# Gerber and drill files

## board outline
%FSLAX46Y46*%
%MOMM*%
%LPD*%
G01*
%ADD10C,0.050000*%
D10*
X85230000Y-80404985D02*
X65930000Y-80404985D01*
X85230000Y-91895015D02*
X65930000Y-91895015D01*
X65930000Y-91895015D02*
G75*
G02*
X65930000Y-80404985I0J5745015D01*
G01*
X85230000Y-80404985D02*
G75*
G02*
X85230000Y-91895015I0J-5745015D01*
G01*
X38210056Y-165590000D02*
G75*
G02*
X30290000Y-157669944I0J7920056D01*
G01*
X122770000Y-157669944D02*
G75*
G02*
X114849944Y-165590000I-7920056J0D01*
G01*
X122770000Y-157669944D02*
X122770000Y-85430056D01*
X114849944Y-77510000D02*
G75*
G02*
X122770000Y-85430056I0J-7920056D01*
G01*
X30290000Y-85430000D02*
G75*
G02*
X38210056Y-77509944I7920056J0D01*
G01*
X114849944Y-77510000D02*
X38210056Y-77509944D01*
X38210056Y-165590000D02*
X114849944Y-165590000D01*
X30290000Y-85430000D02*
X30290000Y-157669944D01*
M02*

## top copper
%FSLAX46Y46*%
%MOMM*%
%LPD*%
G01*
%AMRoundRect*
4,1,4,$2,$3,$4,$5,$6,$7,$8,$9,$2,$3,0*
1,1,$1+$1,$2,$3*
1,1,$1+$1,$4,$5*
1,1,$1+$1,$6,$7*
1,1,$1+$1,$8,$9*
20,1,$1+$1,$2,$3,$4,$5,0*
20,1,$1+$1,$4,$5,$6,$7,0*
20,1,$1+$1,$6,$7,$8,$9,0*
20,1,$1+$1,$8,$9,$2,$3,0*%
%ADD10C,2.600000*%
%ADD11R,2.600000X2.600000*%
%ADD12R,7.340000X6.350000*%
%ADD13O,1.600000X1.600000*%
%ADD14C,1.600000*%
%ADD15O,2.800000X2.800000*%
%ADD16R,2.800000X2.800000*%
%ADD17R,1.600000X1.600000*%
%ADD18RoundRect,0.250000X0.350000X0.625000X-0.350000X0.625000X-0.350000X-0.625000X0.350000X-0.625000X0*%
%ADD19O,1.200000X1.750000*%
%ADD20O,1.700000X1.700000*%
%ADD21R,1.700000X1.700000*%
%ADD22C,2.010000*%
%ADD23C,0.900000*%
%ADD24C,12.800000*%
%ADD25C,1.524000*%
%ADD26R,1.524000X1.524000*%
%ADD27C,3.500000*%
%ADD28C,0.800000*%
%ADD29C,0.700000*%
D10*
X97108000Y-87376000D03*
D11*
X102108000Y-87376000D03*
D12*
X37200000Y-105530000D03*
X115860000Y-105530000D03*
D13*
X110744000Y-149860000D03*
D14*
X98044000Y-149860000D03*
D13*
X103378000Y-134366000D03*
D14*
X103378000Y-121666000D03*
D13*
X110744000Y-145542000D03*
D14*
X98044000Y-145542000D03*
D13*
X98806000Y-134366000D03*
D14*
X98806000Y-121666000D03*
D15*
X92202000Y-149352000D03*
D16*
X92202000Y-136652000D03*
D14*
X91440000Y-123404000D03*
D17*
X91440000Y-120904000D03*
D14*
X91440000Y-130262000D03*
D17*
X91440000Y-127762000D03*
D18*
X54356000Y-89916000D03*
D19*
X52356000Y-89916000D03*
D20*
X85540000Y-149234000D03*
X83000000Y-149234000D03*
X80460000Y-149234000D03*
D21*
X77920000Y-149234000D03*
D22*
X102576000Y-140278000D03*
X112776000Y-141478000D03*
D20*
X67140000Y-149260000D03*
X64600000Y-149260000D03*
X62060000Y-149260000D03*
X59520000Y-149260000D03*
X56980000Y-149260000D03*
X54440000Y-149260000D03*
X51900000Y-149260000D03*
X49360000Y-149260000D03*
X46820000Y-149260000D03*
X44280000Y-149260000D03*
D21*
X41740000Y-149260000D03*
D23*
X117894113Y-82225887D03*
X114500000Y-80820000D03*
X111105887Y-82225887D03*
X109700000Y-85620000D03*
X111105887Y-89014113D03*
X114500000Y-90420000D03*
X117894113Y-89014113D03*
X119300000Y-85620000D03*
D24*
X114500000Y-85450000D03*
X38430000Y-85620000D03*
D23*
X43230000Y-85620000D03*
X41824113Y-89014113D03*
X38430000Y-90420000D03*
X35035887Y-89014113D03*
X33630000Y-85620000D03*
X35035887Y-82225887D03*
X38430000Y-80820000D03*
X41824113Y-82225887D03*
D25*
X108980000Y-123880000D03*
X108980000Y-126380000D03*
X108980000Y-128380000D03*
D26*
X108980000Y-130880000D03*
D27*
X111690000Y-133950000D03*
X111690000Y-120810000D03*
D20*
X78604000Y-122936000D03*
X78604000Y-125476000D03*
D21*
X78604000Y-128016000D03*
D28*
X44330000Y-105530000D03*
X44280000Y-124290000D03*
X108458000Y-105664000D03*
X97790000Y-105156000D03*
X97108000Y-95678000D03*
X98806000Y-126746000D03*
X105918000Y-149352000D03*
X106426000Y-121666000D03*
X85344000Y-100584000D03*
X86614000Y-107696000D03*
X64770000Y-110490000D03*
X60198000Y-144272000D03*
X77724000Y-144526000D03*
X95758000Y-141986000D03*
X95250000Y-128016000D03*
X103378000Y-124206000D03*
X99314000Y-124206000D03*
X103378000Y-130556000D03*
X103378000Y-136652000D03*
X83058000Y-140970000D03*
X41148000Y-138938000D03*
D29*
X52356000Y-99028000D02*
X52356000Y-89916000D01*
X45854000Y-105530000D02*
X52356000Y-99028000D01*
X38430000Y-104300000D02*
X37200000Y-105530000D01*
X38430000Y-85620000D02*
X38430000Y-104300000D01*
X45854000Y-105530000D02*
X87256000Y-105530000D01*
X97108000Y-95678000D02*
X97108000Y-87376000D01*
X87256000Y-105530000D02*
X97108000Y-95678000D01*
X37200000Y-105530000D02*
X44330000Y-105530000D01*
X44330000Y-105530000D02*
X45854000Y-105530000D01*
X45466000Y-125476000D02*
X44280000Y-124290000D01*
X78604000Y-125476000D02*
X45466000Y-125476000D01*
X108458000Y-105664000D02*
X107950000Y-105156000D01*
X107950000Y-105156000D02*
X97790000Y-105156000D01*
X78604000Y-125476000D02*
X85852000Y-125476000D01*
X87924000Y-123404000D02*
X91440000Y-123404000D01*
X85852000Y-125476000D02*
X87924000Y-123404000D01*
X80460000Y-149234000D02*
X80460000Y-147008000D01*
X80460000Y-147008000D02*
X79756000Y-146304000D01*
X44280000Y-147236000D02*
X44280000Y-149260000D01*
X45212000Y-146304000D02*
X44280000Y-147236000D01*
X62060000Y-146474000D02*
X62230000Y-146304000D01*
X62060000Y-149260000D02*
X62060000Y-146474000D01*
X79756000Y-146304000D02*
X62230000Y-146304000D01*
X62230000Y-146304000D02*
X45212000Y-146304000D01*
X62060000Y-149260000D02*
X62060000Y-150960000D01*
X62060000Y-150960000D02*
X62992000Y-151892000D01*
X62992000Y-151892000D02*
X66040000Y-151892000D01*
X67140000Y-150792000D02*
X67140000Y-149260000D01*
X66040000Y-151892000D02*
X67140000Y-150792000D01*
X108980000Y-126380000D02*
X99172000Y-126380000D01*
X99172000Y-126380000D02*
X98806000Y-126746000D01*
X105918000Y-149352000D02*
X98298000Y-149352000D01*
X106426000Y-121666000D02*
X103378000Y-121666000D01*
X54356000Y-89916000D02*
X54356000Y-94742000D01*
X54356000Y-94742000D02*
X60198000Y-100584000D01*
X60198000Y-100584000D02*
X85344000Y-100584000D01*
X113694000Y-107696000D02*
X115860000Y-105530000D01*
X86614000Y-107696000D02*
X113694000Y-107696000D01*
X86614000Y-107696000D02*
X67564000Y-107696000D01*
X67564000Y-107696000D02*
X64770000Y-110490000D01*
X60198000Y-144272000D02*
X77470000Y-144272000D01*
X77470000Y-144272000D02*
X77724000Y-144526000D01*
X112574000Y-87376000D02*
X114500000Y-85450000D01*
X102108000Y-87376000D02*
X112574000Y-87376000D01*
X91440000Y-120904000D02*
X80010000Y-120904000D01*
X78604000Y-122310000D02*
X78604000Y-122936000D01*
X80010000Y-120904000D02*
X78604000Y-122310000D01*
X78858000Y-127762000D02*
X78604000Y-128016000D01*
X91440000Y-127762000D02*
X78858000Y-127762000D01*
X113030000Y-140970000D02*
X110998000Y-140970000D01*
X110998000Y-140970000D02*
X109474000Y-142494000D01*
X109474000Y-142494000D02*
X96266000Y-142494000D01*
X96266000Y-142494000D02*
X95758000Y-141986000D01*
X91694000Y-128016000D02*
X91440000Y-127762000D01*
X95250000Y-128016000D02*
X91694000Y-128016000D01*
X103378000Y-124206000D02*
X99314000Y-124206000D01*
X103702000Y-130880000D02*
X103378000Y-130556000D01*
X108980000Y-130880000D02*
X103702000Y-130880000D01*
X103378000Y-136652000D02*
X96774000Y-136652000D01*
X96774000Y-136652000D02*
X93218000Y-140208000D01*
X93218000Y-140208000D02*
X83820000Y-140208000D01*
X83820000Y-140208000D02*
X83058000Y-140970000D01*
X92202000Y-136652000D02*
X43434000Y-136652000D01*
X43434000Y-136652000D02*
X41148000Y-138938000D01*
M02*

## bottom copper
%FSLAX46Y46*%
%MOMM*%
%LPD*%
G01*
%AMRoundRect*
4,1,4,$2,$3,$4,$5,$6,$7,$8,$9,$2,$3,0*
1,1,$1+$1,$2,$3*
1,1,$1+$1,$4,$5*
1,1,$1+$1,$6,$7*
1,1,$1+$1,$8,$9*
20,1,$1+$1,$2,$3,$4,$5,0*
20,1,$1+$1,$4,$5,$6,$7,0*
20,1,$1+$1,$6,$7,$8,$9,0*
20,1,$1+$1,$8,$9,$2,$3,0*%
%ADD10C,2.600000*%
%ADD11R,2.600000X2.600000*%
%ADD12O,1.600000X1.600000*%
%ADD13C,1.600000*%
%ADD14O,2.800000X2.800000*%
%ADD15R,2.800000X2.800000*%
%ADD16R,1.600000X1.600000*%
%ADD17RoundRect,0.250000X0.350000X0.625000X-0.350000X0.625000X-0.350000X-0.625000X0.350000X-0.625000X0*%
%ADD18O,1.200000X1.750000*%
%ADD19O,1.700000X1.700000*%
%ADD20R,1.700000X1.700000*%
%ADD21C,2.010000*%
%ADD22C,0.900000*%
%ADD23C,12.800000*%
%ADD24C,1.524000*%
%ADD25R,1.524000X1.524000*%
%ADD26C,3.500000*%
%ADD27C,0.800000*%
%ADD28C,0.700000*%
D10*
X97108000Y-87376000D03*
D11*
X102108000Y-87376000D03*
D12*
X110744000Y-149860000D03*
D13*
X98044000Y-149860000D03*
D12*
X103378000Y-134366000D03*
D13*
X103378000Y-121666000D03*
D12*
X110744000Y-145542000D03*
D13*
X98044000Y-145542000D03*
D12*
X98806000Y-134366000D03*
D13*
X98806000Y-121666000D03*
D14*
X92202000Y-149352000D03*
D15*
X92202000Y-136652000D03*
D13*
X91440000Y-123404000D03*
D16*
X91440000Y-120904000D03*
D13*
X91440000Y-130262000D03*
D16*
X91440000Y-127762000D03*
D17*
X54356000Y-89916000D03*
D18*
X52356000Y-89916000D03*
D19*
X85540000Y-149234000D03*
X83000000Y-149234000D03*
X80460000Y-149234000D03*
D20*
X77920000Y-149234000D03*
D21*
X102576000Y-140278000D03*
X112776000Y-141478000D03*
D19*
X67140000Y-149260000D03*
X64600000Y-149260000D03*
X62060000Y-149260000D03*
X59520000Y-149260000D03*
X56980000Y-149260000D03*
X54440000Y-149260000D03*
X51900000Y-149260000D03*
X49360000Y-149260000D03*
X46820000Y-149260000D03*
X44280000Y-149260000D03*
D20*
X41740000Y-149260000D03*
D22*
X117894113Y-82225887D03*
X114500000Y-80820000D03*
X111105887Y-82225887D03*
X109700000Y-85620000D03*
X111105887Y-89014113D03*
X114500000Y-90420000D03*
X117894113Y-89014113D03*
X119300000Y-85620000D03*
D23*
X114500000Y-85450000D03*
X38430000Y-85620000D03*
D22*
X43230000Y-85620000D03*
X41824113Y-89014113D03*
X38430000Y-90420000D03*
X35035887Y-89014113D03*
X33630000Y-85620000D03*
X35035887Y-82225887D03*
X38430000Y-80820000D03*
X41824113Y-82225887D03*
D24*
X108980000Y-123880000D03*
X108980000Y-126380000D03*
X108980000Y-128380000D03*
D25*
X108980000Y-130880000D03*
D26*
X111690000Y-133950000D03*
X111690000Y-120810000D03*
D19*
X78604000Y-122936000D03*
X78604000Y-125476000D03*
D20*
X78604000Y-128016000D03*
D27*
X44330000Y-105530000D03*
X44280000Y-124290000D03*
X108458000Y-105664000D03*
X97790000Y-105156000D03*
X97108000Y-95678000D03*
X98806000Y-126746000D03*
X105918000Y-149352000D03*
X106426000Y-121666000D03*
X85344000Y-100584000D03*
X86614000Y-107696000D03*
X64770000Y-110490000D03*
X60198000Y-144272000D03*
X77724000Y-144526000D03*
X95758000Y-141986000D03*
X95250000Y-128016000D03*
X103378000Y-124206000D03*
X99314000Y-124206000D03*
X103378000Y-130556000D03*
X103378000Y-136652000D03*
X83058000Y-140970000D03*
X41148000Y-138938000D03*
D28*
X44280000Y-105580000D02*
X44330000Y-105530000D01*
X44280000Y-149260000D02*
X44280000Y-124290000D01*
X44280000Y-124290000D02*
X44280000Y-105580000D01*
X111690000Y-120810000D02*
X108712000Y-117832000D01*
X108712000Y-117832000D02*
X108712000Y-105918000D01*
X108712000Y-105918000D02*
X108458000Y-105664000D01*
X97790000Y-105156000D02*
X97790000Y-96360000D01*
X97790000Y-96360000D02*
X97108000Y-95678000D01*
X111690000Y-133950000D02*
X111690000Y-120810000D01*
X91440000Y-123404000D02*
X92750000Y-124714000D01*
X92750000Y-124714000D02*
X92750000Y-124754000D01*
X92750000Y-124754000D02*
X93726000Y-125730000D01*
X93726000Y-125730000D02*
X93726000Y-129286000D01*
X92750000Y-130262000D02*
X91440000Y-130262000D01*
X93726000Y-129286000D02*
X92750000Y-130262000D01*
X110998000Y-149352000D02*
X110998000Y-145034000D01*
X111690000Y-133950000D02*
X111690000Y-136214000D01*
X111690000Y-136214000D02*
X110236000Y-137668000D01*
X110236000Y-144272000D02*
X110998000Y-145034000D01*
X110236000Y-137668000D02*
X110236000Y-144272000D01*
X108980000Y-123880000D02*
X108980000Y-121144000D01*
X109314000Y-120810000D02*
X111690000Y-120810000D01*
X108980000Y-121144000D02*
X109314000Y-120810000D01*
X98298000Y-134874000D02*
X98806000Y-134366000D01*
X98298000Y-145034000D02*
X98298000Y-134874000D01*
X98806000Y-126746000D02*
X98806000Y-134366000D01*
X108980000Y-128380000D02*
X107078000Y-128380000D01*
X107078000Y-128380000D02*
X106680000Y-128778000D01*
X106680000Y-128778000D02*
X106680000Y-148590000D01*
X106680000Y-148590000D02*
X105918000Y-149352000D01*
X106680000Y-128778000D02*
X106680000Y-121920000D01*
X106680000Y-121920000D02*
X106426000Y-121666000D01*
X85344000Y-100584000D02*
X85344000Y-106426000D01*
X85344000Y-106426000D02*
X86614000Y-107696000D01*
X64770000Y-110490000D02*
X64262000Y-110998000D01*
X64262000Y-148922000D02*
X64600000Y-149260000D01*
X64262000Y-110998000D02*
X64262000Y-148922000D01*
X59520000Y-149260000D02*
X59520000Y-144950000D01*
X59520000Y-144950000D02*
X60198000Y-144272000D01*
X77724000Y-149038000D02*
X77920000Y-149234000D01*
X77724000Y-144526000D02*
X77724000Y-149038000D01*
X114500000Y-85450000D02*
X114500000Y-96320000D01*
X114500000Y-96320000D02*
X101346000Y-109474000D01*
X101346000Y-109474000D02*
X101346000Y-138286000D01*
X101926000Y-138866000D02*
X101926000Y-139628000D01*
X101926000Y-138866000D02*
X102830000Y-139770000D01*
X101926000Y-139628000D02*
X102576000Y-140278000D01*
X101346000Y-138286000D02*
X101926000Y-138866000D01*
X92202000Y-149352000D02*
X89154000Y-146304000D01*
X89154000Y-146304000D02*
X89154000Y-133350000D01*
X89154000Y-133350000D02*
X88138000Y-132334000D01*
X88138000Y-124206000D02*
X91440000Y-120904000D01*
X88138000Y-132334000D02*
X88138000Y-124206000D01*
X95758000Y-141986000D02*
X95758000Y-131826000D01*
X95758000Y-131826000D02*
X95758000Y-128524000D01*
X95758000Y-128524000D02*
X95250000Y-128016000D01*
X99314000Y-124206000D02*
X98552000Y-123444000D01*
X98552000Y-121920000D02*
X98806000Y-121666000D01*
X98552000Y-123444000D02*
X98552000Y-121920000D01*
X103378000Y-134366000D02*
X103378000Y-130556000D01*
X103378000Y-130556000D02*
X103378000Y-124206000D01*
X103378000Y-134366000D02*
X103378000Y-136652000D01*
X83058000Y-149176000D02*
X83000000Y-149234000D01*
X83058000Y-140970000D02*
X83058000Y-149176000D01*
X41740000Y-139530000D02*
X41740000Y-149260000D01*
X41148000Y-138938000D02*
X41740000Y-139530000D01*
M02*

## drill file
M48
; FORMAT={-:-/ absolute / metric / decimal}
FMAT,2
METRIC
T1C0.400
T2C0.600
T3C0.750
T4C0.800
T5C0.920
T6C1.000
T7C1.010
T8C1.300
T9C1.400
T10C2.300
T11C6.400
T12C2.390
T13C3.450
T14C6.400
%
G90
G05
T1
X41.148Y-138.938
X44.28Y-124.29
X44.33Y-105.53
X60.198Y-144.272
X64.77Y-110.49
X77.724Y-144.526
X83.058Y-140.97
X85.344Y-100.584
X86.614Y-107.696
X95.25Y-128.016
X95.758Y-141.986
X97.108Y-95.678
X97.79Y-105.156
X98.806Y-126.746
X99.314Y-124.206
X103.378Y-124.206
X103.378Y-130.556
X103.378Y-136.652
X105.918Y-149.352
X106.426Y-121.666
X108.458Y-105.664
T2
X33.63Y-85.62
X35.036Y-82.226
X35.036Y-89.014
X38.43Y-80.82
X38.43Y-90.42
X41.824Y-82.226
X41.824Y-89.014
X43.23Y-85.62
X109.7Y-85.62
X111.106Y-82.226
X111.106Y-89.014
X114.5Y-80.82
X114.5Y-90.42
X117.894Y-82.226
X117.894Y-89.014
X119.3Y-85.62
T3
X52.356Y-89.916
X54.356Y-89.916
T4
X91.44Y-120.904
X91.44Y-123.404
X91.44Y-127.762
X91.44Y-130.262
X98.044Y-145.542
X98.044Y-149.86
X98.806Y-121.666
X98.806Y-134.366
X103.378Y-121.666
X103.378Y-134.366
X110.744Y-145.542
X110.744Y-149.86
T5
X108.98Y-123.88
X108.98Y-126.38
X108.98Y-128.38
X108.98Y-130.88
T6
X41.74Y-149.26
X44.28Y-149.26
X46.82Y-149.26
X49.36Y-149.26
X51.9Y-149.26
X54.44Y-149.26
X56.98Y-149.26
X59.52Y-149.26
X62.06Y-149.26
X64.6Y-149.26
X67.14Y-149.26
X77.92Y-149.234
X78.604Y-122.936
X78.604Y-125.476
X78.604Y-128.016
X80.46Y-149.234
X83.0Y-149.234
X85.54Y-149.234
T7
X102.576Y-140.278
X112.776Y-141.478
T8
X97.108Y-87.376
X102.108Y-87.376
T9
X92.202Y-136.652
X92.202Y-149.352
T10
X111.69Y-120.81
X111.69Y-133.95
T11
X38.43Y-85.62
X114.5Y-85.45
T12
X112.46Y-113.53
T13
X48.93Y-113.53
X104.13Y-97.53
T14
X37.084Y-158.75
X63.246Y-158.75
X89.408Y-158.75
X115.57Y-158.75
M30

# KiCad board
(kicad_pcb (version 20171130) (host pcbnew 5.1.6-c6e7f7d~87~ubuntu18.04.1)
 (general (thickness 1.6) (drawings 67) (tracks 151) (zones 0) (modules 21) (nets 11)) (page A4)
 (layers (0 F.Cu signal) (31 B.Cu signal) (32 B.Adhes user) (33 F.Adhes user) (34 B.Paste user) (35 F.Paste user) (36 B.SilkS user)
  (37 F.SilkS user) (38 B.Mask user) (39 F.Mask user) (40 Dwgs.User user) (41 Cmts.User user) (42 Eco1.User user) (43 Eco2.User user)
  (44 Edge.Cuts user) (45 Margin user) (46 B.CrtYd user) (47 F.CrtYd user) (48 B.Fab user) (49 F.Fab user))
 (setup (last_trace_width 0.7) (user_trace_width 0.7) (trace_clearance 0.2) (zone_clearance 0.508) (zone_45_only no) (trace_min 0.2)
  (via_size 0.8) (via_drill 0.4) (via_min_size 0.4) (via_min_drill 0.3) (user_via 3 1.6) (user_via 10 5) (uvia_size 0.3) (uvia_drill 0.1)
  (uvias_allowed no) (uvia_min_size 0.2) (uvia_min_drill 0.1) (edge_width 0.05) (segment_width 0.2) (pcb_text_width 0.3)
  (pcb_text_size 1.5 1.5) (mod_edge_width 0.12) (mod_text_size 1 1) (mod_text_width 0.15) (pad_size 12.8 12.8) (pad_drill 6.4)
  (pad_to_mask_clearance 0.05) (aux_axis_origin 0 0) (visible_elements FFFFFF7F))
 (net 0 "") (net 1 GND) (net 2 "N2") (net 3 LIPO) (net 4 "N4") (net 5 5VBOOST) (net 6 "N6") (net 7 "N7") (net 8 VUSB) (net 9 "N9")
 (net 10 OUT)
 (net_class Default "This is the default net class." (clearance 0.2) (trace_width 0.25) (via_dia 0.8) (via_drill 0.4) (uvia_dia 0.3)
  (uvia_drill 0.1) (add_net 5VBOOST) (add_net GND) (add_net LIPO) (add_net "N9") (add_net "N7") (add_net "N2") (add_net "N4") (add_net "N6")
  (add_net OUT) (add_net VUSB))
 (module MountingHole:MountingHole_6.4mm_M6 (layer F.Cu) (at 89.408 158.75)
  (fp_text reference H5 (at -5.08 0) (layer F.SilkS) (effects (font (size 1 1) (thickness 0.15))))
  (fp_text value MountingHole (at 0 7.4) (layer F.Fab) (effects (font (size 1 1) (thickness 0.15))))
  (pad 1 np_thru_hole circle (at 0 0) (size 6.4 6.4) (drill 6.4) (layers *.Cu *.Mask)))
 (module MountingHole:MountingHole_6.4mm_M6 (layer F.Cu) (at 63.246 158.75)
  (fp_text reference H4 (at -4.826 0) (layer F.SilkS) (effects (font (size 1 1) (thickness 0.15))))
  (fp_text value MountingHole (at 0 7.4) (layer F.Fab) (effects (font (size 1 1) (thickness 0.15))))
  (pad 1 np_thru_hole circle (at 0 0) (size 6.4 6.4) (drill 6.4) (layers *.Cu *.Mask)))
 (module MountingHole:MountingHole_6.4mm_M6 (layer F.Cu) (at 115.57 158.75)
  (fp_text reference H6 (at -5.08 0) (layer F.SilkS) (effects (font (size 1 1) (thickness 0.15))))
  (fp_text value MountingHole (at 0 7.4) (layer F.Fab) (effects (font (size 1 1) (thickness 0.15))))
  (pad 1 np_thru_hole circle (at 0 0) (size 6.4 6.4) (drill 6.4) (layers *.Cu *.Mask)))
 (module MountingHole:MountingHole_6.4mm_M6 (layer F.Cu) (at 37.084 158.75)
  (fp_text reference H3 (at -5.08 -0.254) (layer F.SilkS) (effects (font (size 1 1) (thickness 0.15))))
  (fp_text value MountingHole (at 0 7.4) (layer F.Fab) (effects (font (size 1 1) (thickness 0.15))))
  (pad 1 np_thru_hole circle (at 0 0) (size 6.4 6.4) (drill 6.4) (layers *.Cu *.Mask)))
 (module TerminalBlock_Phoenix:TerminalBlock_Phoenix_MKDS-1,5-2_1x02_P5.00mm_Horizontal (layer F.Cu) (at 102.108 87.376 180)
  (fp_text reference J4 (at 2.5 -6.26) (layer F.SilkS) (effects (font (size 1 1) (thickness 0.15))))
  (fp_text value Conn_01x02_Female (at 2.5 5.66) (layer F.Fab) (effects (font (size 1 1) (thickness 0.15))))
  (pad 2 thru_hole circle (at 5 0 180) (size 2.6 2.6) (drill 1.3) (layers *.Cu *.Mask) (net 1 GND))
  (pad 1 thru_hole rect (at 0 0 180) (size 2.6 2.6) (drill 1.3) (layers *.Cu *.Mask) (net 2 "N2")))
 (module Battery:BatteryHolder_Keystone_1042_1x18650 (layer F.Cu) (at 76.53 105.53 180)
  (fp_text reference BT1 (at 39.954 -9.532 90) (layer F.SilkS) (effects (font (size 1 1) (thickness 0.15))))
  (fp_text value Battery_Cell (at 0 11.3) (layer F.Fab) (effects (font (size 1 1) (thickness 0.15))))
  (pad "" np_thru_hole circle (at -35.93 -8 180) (size 2.39 2.39) (drill 2.39) (layers *.Cu *.Mask))
  (pad "" np_thru_hole circle (at -27.6 8 180) (size 3.45 3.45) (drill 3.45) (layers *.Cu *.Mask))
  (pad "" np_thru_hole circle (at 27.6 -8 180) (size 3.45 3.45) (drill 3.45) (layers *.Cu *.Mask))
  (pad 2 smd rect (at 39.33 0 180) (size 7.34 6.35) (layers F.Cu F.Paste F.Mask) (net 1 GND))
  (pad 1 smd rect (at -39.33 0 180) (size 7.34 6.35) (layers F.Cu F.Paste F.Mask) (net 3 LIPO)))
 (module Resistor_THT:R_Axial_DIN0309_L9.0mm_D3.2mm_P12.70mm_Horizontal (layer F.Cu) (at 98.044 149.86)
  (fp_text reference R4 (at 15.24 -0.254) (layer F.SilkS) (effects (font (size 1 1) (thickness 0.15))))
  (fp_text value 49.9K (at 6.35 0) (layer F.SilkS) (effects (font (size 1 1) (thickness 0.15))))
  (pad 2 thru_hole oval (at 12.7 0) (size 1.6 1.6) (drill 0.8) (layers *.Cu *.Mask) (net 1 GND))
  (pad 1 thru_hole circle (at 0 0) (size 1.6 1.6) (drill 0.8) (layers *.Cu *.Mask) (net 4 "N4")))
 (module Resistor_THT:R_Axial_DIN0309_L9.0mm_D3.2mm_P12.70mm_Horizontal (layer F.Cu) (at 103.378 121.666 270)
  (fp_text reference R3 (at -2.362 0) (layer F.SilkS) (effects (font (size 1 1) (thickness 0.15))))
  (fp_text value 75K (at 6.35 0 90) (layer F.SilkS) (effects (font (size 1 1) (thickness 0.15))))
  (pad 2 thru_hole oval (at 12.7 0 270) (size 1.6 1.6) (drill 0.8) (layers *.Cu *.Mask) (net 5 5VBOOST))
  (pad 1 thru_hole circle (at 0 0 270) (size 1.6 1.6) (drill 0.8) (layers *.Cu *.Mask) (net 4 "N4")))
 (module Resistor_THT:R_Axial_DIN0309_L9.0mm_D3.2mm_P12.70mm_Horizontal (layer F.Cu) (at 98.044 145.542)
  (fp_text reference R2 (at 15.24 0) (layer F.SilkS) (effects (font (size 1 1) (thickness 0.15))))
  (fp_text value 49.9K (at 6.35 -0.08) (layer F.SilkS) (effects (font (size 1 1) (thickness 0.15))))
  (pad 2 thru_hole oval (at 12.7 0) (size 1.6 1.6) (drill 0.8) (layers *.Cu *.Mask) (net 1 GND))
  (pad 1 thru_hole circle (at 0 0) (size 1.6 1.6) (drill 0.8) (layers *.Cu *.Mask) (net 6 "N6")))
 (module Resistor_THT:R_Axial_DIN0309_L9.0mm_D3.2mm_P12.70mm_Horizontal (layer F.Cu) (at 98.806 121.666 270)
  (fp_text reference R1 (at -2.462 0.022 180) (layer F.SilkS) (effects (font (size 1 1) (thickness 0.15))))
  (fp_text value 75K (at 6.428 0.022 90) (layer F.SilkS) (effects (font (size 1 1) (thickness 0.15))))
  (pad 2 thru_hole oval (at 12.7 0 270) (size 1.6 1.6) (drill 0.8) (layers *.Cu *.Mask) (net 6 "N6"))
  (pad 1 thru_hole circle (at 0 0 270) (size 1.6 1.6) (drill 0.8) (layers *.Cu *.Mask) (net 5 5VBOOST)))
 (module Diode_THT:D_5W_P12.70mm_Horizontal (layer F.Cu) (at 92.202 136.652 270)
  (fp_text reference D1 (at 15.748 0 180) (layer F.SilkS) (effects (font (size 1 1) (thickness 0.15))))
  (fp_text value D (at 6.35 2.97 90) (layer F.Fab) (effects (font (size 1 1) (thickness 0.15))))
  (pad 2 thru_hole oval (at 12.7 0 270) (size 2.8 2.8) (drill 1.4) (layers *.Cu *.Mask) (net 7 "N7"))
  (pad 1 thru_hole rect (at 0 0 270) (size 2.8 2.8) (drill 1.4) (layers *.Cu *.Mask) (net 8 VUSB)))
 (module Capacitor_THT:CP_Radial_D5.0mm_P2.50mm (layer F.Cu) (at 91.44 120.904 270)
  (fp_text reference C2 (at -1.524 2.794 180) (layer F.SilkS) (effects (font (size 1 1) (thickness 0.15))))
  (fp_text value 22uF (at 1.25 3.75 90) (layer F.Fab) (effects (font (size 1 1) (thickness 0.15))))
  (pad 2 thru_hole circle (at 2.5 0 270) (size 1.6 1.6) (drill 0.8) (layers *.Cu *.Mask) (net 1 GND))
  (pad 1 thru_hole rect (at 0 0 270) (size 1.6 1.6) (drill 0.8) (layers *.Cu *.Mask) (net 7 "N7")))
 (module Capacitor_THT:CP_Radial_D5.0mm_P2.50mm (layer F.Cu) (at 91.44 127.762 270)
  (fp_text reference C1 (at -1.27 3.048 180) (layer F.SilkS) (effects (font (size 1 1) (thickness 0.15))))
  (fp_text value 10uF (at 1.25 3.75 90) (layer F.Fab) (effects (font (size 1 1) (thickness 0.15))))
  (pad 2 thru_hole circle (at 2.5 0 270) (size 1.6 1.6) (drill 0.8) (layers *.Cu *.Mask) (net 1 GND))
  (pad 1 thru_hole rect (at 0 0 270) (size 1.6 1.6) (drill 0.8) (layers *.Cu *.Mask) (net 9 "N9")))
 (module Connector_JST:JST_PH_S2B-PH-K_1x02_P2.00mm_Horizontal (layer F.Cu) (at 54.356 89.916 180)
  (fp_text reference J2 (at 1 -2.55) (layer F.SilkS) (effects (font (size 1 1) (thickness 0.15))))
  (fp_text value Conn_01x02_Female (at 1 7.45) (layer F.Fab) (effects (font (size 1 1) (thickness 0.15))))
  (pad 1 thru_hole roundrect (at 0 0 180) (size 1.2 1.75) (drill 0.75) (layers *.Cu *.Mask) (roundrect_rratio 0.208333) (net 3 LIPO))
  (pad 2 thru_hole oval (at 2 0 180) (size 1.2 1.75) (drill 0.75) (layers *.Cu *.Mask) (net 1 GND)))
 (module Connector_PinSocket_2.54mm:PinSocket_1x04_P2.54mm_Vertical (layer F.Cu) (at 77.92 149.234 90)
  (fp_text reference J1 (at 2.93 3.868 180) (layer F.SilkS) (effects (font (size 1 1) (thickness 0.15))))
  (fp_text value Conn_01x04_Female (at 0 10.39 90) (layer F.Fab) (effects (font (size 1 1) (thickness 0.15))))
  (pad 4 thru_hole oval (at 0 7.62 90) (size 1.7 1.7) (drill 1) (layers *.Cu *.Mask))
  (pad 3 thru_hole oval (at 0 5.08 90) (size 1.7 1.7) (drill 1) (layers *.Cu *.Mask) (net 5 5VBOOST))
  (pad 2 thru_hole oval (at 0 2.54 90) (size 1.7 1.7) (drill 1) (layers *.Cu *.Mask) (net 1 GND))
  (pad 1 thru_hole rect (at 0 0 90) (size 1.7 1.7) (drill 1) (layers *.Cu *.Mask) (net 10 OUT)))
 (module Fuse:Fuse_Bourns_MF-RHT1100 (layer F.Cu) (at 112.776 141.478 180)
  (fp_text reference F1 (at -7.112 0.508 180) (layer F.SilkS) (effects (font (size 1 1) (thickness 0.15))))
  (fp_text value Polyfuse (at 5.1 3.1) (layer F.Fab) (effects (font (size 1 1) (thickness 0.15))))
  (pad 2 thru_hole circle (at 10.2 1.2 180) (size 2.01 2.01) (drill 1.01) (layers *.Cu *.Mask) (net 2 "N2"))
  (pad 1 thru_hole circle (at 0 0 180) (size 2.01 2.01) (drill 1.01) (layers *.Cu *.Mask) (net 9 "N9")))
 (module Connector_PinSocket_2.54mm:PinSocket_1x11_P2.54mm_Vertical (layer F.Cu) (at 41.74 149.26 90)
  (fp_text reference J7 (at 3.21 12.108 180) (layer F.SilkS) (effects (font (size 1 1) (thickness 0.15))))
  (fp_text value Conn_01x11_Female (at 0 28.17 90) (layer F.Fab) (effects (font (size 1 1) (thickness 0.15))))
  (pad 11 thru_hole oval (at 0 25.4 90) (size 1.7 1.7) (drill 1) (layers *.Cu *.Mask) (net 1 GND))
  (pad 10 thru_hole oval (at 0 22.86 90) (size 1.7 1.7) (drill 1) (layers *.Cu *.Mask) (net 3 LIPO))
  (pad 9 thru_hole oval (at 0 20.32 90) (size 1.7 1.7) (drill 1) (layers *.Cu *.Mask) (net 1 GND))
  (pad 8 thru_hole oval (at 0 17.78 90) (size 1.7 1.7) (drill 1) (layers *.Cu *.Mask) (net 10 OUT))
  (pad 7 thru_hole oval (at 0 15.24 90) (size 1.7 1.7) (drill 1) (layers *.Cu *.Mask))
  (pad 6 thru_hole oval (at 0 12.7 90) (size 1.7 1.7) (drill 1) (layers *.Cu *.Mask))
  (pad 5 thru_hole oval (at 0 10.16 90) (size 1.7 1.7) (drill 1) (layers *.Cu *.Mask))
  (pad 4 thru_hole oval (at 0 7.62 90) (size 1.7 1.7) (drill 1) (layers *.Cu *.Mask))
  (pad 3 thru_hole oval (at 0 5.08 90) (size 1.7 1.7) (drill 1) (layers *.Cu *.Mask))
  (pad 2 thru_hole oval (at 0 2.54 90) (size 1.7 1.7) (drill 1) (layers *.Cu *.Mask) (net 1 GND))
  (pad 1 thru_hole rect (at 0 0 90) (size 1.7 1.7) (drill 1) (layers *.Cu *.Mask) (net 8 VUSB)))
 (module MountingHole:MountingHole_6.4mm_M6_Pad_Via (layer F.Cu) (at 114.5 85.62)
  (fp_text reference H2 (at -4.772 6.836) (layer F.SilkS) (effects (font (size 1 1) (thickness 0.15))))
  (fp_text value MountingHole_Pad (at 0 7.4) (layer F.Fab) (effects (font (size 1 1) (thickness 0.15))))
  (pad 1 thru_hole circle (at 3.394113 -3.394113) (size 0.9 0.9) (drill 0.6) (layers *.Cu *.Mask) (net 2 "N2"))
  (pad 1 thru_hole circle (at 0 -4.8) (size 0.9 0.9) (drill 0.6) (layers *.Cu *.Mask) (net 2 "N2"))
  (pad 1 thru_hole circle (at -3.394113 -3.394113) (size 0.9 0.9) (drill 0.6) (layers *.Cu *.Mask) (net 2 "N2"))
  (pad 1 thru_hole circle (at -4.8 0) (size 0.9 0.9) (drill 0.6) (layers *.Cu *.Mask) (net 2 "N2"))
  (pad 1 thru_hole circle (at -3.394113 3.394113) (size 0.9 0.9) (drill 0.6) (layers *.Cu *.Mask) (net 2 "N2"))
  (pad 1 thru_hole circle (at 0 4.8) (size 0.9 0.9) (drill 0.6) (layers *.Cu *.Mask) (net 2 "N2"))
  (pad 1 thru_hole circle (at 3.394113 3.394113) (size 0.9 0.9) (drill 0.6) (layers *.Cu *.Mask) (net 2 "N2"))
  (pad 1 thru_hole circle (at 4.8 0) (size 0.9 0.9) (drill 0.6) (layers *.Cu *.Mask) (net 2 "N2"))
  (pad 1 thru_hole circle (at 0 -0.17) (size 12.8 12.8) (drill 6.4) (layers *.Cu *.Mask) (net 2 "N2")))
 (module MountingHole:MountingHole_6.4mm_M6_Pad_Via (layer F.Cu) (at 38.43 85.62)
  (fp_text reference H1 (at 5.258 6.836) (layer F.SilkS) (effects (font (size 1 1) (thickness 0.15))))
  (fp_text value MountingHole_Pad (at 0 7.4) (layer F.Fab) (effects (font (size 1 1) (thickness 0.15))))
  (pad 1 thru_hole circle (at 0 0) (size 12.8 12.8) (drill 6.4) (layers *.Cu *.Mask) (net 1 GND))
  (pad 1 thru_hole circle (at 4.8 0) (size 0.9 0.9) (drill 0.6) (layers *.Cu *.Mask) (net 1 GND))
  (pad 1 thru_hole circle (at 3.394113 3.394113) (size 0.9 0.9) (drill 0.6) (layers *.Cu *.Mask) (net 1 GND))
  (pad 1 thru_hole circle (at 0 4.8) (size 0.9 0.9) (drill 0.6) (layers *.Cu *.Mask) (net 1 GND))
  (pad 1 thru_hole circle (at -3.394113 3.394113) (size 0.9 0.9) (drill 0.6) (layers *.Cu *.Mask) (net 1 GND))
  (pad 1 thru_hole circle (at -4.8 0) (size 0.9 0.9) (drill 0.6) (layers *.Cu *.Mask) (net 1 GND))
  (pad 1 thru_hole circle (at -3.394113 -3.394113) (size 0.9 0.9) (drill 0.6) (layers *.Cu *.Mask) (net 1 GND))
  (pad 1 thru_hole circle (at 0 -4.8) (size 0.9 0.9) (drill 0.6) (layers *.Cu *.Mask) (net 1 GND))
  (pad 1 thru_hole circle (at 3.394113 -3.394113) (size 0.9 0.9) (drill 0.6) (layers *.Cu *.Mask) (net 1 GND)))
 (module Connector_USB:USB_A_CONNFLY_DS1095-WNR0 (layer F.Cu) (at 108.98 130.88 90)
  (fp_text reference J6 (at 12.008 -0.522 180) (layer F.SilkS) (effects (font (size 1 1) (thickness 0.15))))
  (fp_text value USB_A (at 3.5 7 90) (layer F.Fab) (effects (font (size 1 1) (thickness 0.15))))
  (pad 4 thru_hole circle (at 7 0 90) (size 1.524 1.524) (drill 0.92) (layers *.Cu *.Mask) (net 1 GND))
  (pad 3 thru_hole circle (at 4.5 0 90) (size 1.524 1.524) (drill 0.92) (layers *.Cu *.Mask) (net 6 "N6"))
  (pad 2 thru_hole circle (at 2.5 0 90) (size 1.524 1.524) (drill 0.92) (layers *.Cu *.Mask) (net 4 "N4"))
  (pad 1 thru_hole rect (at 0 0 90) (size 1.524 1.524) (drill 0.92) (layers *.Cu *.Mask) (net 5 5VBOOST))
  (pad 5 thru_hole circle (at -3.07 2.71 90) (size 3.5 3.5) (drill 2.3) (layers *.Cu *.Mask) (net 1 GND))
  (pad 5 thru_hole circle (at 10.07 2.71 90) (size 3.5 3.5) (drill 2.3) (layers *.Cu *.Mask) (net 1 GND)))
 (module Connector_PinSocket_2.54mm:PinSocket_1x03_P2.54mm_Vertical (layer F.Cu) (at 78.604 128.016 180)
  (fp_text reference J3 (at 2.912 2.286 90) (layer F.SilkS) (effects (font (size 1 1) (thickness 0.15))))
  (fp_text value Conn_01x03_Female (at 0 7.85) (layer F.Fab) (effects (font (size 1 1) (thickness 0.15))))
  (pad 3 thru_hole oval (at 0 5.08 180) (size 1.7 1.7) (drill 1) (layers *.Cu *.Mask) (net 7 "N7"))
  (pad 2 thru_hole oval (at 0 2.54 180) (size 1.7 1.7) (drill 1) (layers *.Cu *.Mask) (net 1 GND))
  (pad 1 thru_hole rect (at 0 0 180) (size 1.7 1.7) (drill 1) (layers *.Cu *.Mask) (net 9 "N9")))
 (gr_line (start 85.23 80.404985) (end 65.93 80.404985) (layer Edge.Cuts) (width 0.05))
 (gr_line (start 85.23 91.895015) (end 65.93 91.895015) (layer Edge.Cuts) (width 0.05))
 (gr_arc (start 65.93 86.15) (end 65.93 80.404985) (angle -180) (layer Edge.Cuts) (width 0.05))
 (gr_arc (start 85.23 86.15) (end 85.23 91.895015) (angle -180) (layer Edge.Cuts) (width 0.05))
 (gr_arc (start 38.210056 157.669944) (end 30.29 157.669944) (angle -90) (layer Edge.Cuts) (width 0.05))
 (gr_arc (start 114.849944 157.669944) (end 114.849944 165.59) (angle -90) (layer Edge.Cuts) (width 0.05))
 (gr_line (start 122.77 157.669944) (end 122.77 85.430056) (layer Edge.Cuts) (width 0.05))
 (gr_arc (start 114.849944 85.430056) (end 122.77 85.430056) (angle -90) (layer Edge.Cuts) (width 0.05))
 (gr_arc (start 38.210056 85.43) (end 38.210056 77.509944) (angle -90) (layer Edge.Cuts) (width 0.05))
 (gr_line (start 114.849944 77.51) (end 38.210056 77.509944) (layer Edge.Cuts) (width 0.05))
 (gr_line (start 38.210056 165.59) (end 114.849944 165.59) (layer Edge.Cuts) (width 0.05))
 (gr_line (start 30.29 85.43) (end 30.29 157.669944) (layer Edge.Cuts) (width 0.05))
 (segment (start 52.356 99.028) (end 52.356 89.916) (width 0.7) (layer F.Cu) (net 1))
 (segment (start 45.854 105.53) (end 52.356 99.028) (width 0.7) (layer F.Cu) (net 1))
 (segment (start 38.43 104.3) (end 37.2 105.53) (width 0.7) (layer F.Cu) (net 1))
 (segment (start 38.43 85.62) (end 38.43 104.3) (width 0.7) (layer F.Cu) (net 1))
 (segment (start 45.854 105.53) (end 87.256 105.53) (width 0.7) (layer F.Cu) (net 1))
 (segment (start 97.108 95.678) (end 97.108 87.376) (width 0.7) (layer F.Cu) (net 1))
 (segment (start 87.256 105.53) (end 97.108 95.678) (width 0.7) (layer F.Cu) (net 1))
 (via (at 44.33 105.53) (size 0.8) (drill 0.4) (layers F.Cu B.Cu) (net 1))
 (segment (start 44.28 105.58) (end 44.33 105.53) (width 0.7) (layer B.Cu) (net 1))
 (segment (start 37.2 105.53) (end 44.33 105.53) (width 0.7) (layer F.Cu) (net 1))
 (segment (start 44.33 105.53) (end 45.854 105.53) (width 0.7) (layer F.Cu) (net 1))
 (via (at 44.28 124.29) (size 0.8) (drill 0.4) (layers F.Cu B.Cu) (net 1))
 (segment (start 44.28 149.26) (end 44.28 124.29) (width 0.7) (layer B.Cu) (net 1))
 (segment (start 45.466 125.476) (end 44.28 124.29) (width 0.7) (layer F.Cu) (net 1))
 (segment (start 78.604 125.476) (end 45.466 125.476) (width 0.7) (layer F.Cu) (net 1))
 (segment (start 44.28 124.29) (end 44.28 105.58) (width 0.7) (layer B.Cu) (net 1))
 (segment (start 111.69 120.81) (end 108.712 117.832) (width 0.7) (layer B.Cu) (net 1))
 (via (at 108.458 105.664) (size 0.8) (drill 0.4) (layers F.Cu B.Cu) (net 1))
 (segment (start 108.712 117.832) (end 108.712 105.918) (width 0.7) (layer B.Cu) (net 1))
 (segment (start 108.712 105.918) (end 108.458 105.664) (width 0.7) (layer B.Cu) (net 1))
 (segment (start 108.458 105.664) (end 107.95 105.156) (width 0.7) (layer F.Cu) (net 1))
 (via (at 97.79 105.156) (size 0.8) (drill 0.4) (layers F.Cu B.Cu) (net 1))
 (segment (start 107.95 105.156) (end 97.79 105.156) (width 0.7) (layer F.Cu) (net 1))
 (via (at 97.108 95.678) (size 0.8) (drill 0.4) (layers F.Cu B.Cu) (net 1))
 (segment (start 97.79 105.156) (end 97.79 96.36) (width 0.7) (layer B.Cu) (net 1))
 (segment (start 97.79 96.36) (end 97.108 95.678) (width 0.7) (layer B.Cu) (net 1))
 (segment (start 111.69 133.95) (end 111.69 120.81) (width 0.7) (layer B.Cu) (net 1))
 (segment (start 78.604 125.476) (end 85.852 125.476) (width 0.7) (layer F.Cu) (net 1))
 (segment (start 87.924 123.404) (end 91.44 123.404) (width 0.7) (layer F.Cu) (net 1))
 (segment (start 85.852 125.476) (end 87.924 123.404) (width 0.7) (layer F.Cu) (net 1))
 (segment (start 91.44 123.404) (end 92.75 124.714) (width 0.7) (layer B.Cu) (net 1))
 (segment (start 92.75 124.714) (end 92.75 124.754) (width 0.7) (layer B.Cu) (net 1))
 (segment (start 92.75 124.754) (end 93.726 125.73) (width 0.7) (layer B.Cu) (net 1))
 (segment (start 93.726 125.73) (end 93.726 129.286) (width 0.7) (layer B.Cu) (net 1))
 (segment (start 92.75 130.262) (end 91.44 130.262) (width 0.7) (layer B.Cu) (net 1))
 (segment (start 93.726 129.286) (end 92.75 130.262) (width 0.7) (layer B.Cu) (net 1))
 (segment (start 80.46 149.234) (end 80.46 147.008) (width 0.7) (layer F.Cu) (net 1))
 (segment (start 80.46 147.008) (end 79.756 146.304) (width 0.7) (layer F.Cu) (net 1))
 (segment (start 44.28 147.236) (end 44.28 149.26) (width 0.7) (layer F.Cu) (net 1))
 (segment (start 45.212 146.304) (end 44.28 147.236) (width 0.7) (layer F.Cu) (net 1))
 (segment (start 62.06 146.474) (end 62.23 146.304) (width 0.7) (layer F.Cu) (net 1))
 (segment (start 62.06 149.26) (end 62.06 146.474) (width 0.7) (layer F.Cu) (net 1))
 (segment (start 79.756 146.304) (end 62.23 146.304) (width 0.7) (layer F.Cu) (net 1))
 (segment (start 62.23 146.304) (end 45.212 146.304) (width 0.7) (layer F.Cu) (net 1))
 (segment (start 110.998 149.352) (end 110.998 145.034) (width 0.7) (layer B.Cu) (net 1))
 (segment (start 111.69 133.95) (end 111.69 136.214) (width 0.7) (layer B.Cu) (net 1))
 (segment (start 111.69 136.214) (end 110.236 137.668) (width 0.7) (layer B.Cu) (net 1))
 (segment (start 110.236 144.272) (end 110.998 145.034) (width 0.7) (layer B.Cu) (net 1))
 (segment (start 110.236 137.668) (end 110.236 144.272) (width 0.7) (layer B.Cu) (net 1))
 (segment (start 108.98 123.88) (end 108.98 121.144) (width 0.7) (layer B.Cu) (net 1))
 (segment (start 109.314 120.81) (end 111.69 120.81) (width 0.7) (layer B.Cu) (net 1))
 (segment (start 108.98 121.144) (end 109.314 120.81) (width 0.7) (layer B.Cu) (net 1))
 (segment (start 62.06 149.26) (end 62.06 150.96) (width 0.7) (layer F.Cu) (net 1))
 (segment (start 62.06 150.96) (end 62.992 151.892) (width 0.7) (layer F.Cu) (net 1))
 (segment (start 62.992 151.892) (end 66.04 151.892) (width 0.7) (layer F.Cu) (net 1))
 (segment (start 67.14 150.792) (end 67.14 149.26) (width 0.7) (layer F.Cu) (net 1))
 (segment (start 66.04 151.892) (end 67.14 150.792) (width 0.7) (layer F.Cu) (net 1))
 (segment (start 98.298 134.874) (end 98.806 134.366) (width 0.7) (layer B.Cu) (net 6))
 (segment (start 98.298 145.034) (end 98.298 134.874) (width 0.7) (layer B.Cu) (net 6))
 (segment (start 108.98 126.38) (end 99.172 126.38) (width 0.7) (layer F.Cu) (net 6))
 (via (at 98.806 126.746) (size 0.8) (drill 0.4) (layers F.Cu B.Cu) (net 6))
 (segment (start 99.172 126.38) (end 98.806 126.746) (width 0.7) (layer F.Cu) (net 6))
 (segment (start 98.806 126.746) (end 98.806 134.366) (width 0.7) (layer B.Cu) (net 6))
 (segment (start 108.98 128.38) (end 107.078 128.38) (width 0.7) (layer B.Cu) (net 4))
 (segment (start 107.078 128.38) (end 106.68 128.778) (width 0.7) (layer B.Cu) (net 4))
 (via (at 105.918 149.352) (size 0.8) (drill 0.4) (layers F.Cu B.Cu) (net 4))
 (segment (start 106.68 128.778) (end 106.68 148.59) (width 0.7) (layer B.Cu) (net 4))
 (segment (start 106.68 148.59) (end 105.918 149.352) (width 0.7) (layer B.Cu) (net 4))
 (segment (start 105.918 149.352) (end 98.298 149.352) (width 0.7) (layer F.Cu) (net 4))
 (via (at 106.426 121.666) (size 0.8) (drill 0.4) (layers F.Cu B.Cu) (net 4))
 (segment (start 106.68 128.778) (end 106.68 121.92) (width 0.7) (layer B.Cu) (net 4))
 (segment (start 106.68 121.92) (end 106.426 121.666) (width 0.7) (layer B.Cu) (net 4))
 (segment (start 106.426 121.666) (end 103.378 121.666) (width 0.7) (layer F.Cu) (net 4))
 (segment (start 54.356 89.916) (end 54.356 94.742) (width 0.7) (layer F.Cu) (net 3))
 (via (at 85.344 100.584) (size 0.8) (drill 0.4) (layers F.Cu B.Cu) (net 3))
 (segment (start 54.356 94.742) (end 60.198 100.584) (width 0.7) (layer F.Cu) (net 3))
 (segment (start 60.198 100.584) (end 85.344 100.584) (width 0.7) (layer F.Cu) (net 3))
 (via (at 86.614 107.696) (size 0.8) (drill 0.4) (layers F.Cu B.Cu) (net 3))
 (segment (start 85.344 100.584) (end 85.344 106.426) (width 0.7) (layer B.Cu) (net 3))
 (segment (start 85.344 106.426) (end 86.614 107.696) (width 0.7) (layer B.Cu) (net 3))
 (segment (start 113.694 107.696) (end 115.86 105.53) (width 0.7) (layer F.Cu) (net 3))
 (segment (start 86.614 107.696) (end 113.694 107.696) (width 0.7) (layer F.Cu) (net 3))
 (via (at 64.77 110.49) (size 0.8) (drill 0.4) (layers F.Cu B.Cu) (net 3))
 (segment (start 86.614 107.696) (end 67.564 107.696) (width 0.7) (layer F.Cu) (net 3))
 (segment (start 67.564 107.696) (end 64.77 110.49) (width 0.7) (layer F.Cu) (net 3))
 (segment (start 64.77 110.49) (end 64.262 110.998) (width 0.7) (layer B.Cu) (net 3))
 (segment (start 64.262 148.922) (end 64.6 149.26) (width 0.7) (layer B.Cu) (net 3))
 (segment (start 64.262 110.998) (end 64.262 148.922) (width 0.7) (layer B.Cu) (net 3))
 (via (at 60.198 144.272) (size 0.8) (drill 0.4) (layers F.Cu B.Cu) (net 10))
 (segment (start 59.52 149.26) (end 59.52 144.95) (width 0.7) (layer B.Cu) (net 10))
 (segment (start 59.52 144.95) (end 60.198 144.272) (width 0.7) (layer B.Cu) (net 10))
 (via (at 77.724 144.526) (size 0.8) (drill 0.4) (layers F.Cu B.Cu) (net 10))
 (segment (start 60.198 144.272) (end 77.47 144.272) (width 0.7) (layer F.Cu) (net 10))
 (segment (start 77.47 144.272) (end 77.724 144.526) (width 0.7) (layer F.Cu) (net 10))
 (segment (start 77.724 149.038) (end 77.92 149.234) (width 0.7) (layer B.Cu) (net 10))
 (segment (start 77.724 144.526) (end 77.724 149.038) (width 0.7) (layer B.Cu) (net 10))
 (segment (start 112.574 87.376) (end 114.5 85.45) (width 0.7) (layer F.Cu) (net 2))
 (segment (start 102.108 87.376) (end 112.574 87.376) (width 0.7) (layer F.Cu) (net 2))
 (segment (start 114.5 85.45) (end 114.5 96.32) (width 0.7) (layer B.Cu) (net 2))
 (segment (start 114.5 96.32) (end 101.346 109.474) (width 0.7) (layer B.Cu) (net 2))
 (segment (start 101.346 109.474) (end 101.346 138.286) (width 0.7) (layer B.Cu) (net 2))
 (segment (start 101.926 138.866) (end 101.926 139.628) (width 0.7) (layer B.Cu) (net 2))
 (segment (start 101.926 138.866) (end 102.83 139.77) (width 0.7) (layer B.Cu) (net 2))
 (segment (start 101.926 139.628) (end 102.576 140.278) (width 0.7) (layer B.Cu) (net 2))
 (segment (start 101.346 138.286) (end 101.926 138.866) (width 0.7) (layer B.Cu) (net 2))
 (segment (start 91.44 120.904) (end 80.01 120.904) (width 0.7) (layer F.Cu) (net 7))
 (segment (start 78.604 122.31) (end 78.604 122.936) (width 0.7) (layer F.Cu) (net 7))
 (segment (start 80.01 120.904) (end 78.604 122.31) (width 0.7) (layer F.Cu) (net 7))
 (segment (start 92.202 149.352) (end 89.154 146.304) (width 0.7) (layer B.Cu) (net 7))
 (segment (start 89.154 146.304) (end 89.154 133.35) (width 0.7) (layer B.Cu) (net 7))
 (segment (start 89.154 133.35) (end 88.138 132.334) (width 0.7) (layer B.Cu) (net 7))
 (segment (start 88.138 124.206) (end 91.44 120.904) (width 0.7) (layer B.Cu) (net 7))
 (segment (start 88.138 132.334) (end 88.138 124.206) (width 0.7) (layer B.Cu) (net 7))
 (segment (start 78.858 127.762) (end 78.604 128.016) (width 0.7) (layer F.Cu) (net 9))
 (segment (start 91.44 127.762) (end 78.858 127.762) (width 0.7) (layer F.Cu) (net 9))
 (segment (start 113.03 140.97) (end 110.998 140.97) (width 0.7) (layer F.Cu) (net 9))
 (segment (start 110.998 140.97) (end 109.474 142.494) (width 0.7) (layer F.Cu) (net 9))
 (via (at 95.758 141.986) (size 0.8) (drill 0.4) (layers F.Cu B.Cu) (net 9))
 (segment (start 109.474 142.494) (end 96.266 142.494) (width 0.7) (layer F.Cu) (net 9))
 (segment (start 96.266 142.494) (end 95.758 141.986) (width 0.7) (layer F.Cu) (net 9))
 (segment (start 95.758 141.986) (end 95.758 131.826) (width 0.7) (layer B.Cu) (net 9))
 (segment (start 95.758 131.826) (end 95.758 128.524) (width 0.7) (layer B.Cu) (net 9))
 (via (at 95.25 128.016) (size 0.8) (drill 0.4) (layers F.Cu B.Cu) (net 9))
 (segment (start 95.758 128.524) (end 95.25 128.016) (width 0.7) (layer B.Cu) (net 9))
 (segment (start 91.694 128.016) (end 91.44 127.762) (width 0.7) (layer F.Cu) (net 9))
 (segment (start 95.25 128.016) (end 91.694 128.016) (width 0.7) (layer F.Cu) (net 9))
 (via (at 103.378 124.206) (size 0.8) (drill 0.4) (layers F.Cu B.Cu) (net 5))
 (segment (start 103.378 124.206) (end 99.314 124.206) (width 0.7) (layer F.Cu) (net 5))
 (via (at 99.314 124.206) (size 0.8) (drill 0.4) (layers F.Cu B.Cu) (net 5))
 (segment (start 99.314 124.206) (end 98.552 123.444) (width 0.7) (layer B.Cu) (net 5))
 (segment (start 98.552 121.92) (end 98.806 121.666) (width 0.7) (layer B.Cu) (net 5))
 (segment (start 98.552 123.444) (end 98.552 121.92) (width 0.7) (layer B.Cu) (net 5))
 (via (at 103.378 130.556) (size 0.8) (drill 0.4) (layers F.Cu B.Cu) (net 5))
 (segment (start 103.702 130.88) (end 103.378 130.556) (width 0.7) (layer F.Cu) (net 5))
 (segment (start 108.98 130.88) (end 103.702 130.88) (width 0.7) (layer F.Cu) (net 5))
 (segment (start 103.378 134.366) (end 103.378 130.556) (width 0.7) (layer B.Cu) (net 5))
 (segment (start 103.378 130.556) (end 103.378 124.206) (width 0.7) (layer B.Cu) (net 5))
 (via (at 103.378 136.652) (size 0.8) (drill 0.4) (layers F.Cu B.Cu) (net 5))
 (segment (start 103.378 134.366) (end 103.378 136.652) (width 0.7) (layer B.Cu) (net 5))
 (segment (start 103.378 136.652) (end 96.774 136.652) (width 0.7) (layer F.Cu) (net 5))
 (segment (start 96.774 136.652) (end 93.218 140.208) (width 0.7) (layer F.Cu) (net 5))
 (segment (start 93.218 140.208) (end 83.82 140.208) (width 0.7) (layer F.Cu) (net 5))
 (via (at 83.058 140.97) (size 0.8) (drill 0.4) (layers F.Cu B.Cu) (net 5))
 (segment (start 83.82 140.208) (end 83.058 140.97) (width 0.7) (layer F.Cu) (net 5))
 (segment (start 83.058 149.176) (end 83 149.234) (width 0.7) (layer B.Cu) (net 5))
 (segment (start 83.058 140.97) (end 83.058 149.176) (width 0.7) (layer B.Cu) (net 5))
 (via (at 41.148 138.938) (size 0.8) (drill 0.4) (layers F.Cu B.Cu) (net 8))
 (segment (start 92.202 136.652) (end 43.434 136.652) (width 0.7) (layer F.Cu) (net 8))
 (segment (start 43.434 136.652) (end 41.148 138.938) (width 0.7) (layer F.Cu) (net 8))
 (segment (start 41.74 139.53) (end 41.74 149.26) (width 0.7) (layer B.Cu) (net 8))
 (segment (start 41.148 138.938) (end 41.74 139.53) (width 0.7) (layer B.Cu) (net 8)))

